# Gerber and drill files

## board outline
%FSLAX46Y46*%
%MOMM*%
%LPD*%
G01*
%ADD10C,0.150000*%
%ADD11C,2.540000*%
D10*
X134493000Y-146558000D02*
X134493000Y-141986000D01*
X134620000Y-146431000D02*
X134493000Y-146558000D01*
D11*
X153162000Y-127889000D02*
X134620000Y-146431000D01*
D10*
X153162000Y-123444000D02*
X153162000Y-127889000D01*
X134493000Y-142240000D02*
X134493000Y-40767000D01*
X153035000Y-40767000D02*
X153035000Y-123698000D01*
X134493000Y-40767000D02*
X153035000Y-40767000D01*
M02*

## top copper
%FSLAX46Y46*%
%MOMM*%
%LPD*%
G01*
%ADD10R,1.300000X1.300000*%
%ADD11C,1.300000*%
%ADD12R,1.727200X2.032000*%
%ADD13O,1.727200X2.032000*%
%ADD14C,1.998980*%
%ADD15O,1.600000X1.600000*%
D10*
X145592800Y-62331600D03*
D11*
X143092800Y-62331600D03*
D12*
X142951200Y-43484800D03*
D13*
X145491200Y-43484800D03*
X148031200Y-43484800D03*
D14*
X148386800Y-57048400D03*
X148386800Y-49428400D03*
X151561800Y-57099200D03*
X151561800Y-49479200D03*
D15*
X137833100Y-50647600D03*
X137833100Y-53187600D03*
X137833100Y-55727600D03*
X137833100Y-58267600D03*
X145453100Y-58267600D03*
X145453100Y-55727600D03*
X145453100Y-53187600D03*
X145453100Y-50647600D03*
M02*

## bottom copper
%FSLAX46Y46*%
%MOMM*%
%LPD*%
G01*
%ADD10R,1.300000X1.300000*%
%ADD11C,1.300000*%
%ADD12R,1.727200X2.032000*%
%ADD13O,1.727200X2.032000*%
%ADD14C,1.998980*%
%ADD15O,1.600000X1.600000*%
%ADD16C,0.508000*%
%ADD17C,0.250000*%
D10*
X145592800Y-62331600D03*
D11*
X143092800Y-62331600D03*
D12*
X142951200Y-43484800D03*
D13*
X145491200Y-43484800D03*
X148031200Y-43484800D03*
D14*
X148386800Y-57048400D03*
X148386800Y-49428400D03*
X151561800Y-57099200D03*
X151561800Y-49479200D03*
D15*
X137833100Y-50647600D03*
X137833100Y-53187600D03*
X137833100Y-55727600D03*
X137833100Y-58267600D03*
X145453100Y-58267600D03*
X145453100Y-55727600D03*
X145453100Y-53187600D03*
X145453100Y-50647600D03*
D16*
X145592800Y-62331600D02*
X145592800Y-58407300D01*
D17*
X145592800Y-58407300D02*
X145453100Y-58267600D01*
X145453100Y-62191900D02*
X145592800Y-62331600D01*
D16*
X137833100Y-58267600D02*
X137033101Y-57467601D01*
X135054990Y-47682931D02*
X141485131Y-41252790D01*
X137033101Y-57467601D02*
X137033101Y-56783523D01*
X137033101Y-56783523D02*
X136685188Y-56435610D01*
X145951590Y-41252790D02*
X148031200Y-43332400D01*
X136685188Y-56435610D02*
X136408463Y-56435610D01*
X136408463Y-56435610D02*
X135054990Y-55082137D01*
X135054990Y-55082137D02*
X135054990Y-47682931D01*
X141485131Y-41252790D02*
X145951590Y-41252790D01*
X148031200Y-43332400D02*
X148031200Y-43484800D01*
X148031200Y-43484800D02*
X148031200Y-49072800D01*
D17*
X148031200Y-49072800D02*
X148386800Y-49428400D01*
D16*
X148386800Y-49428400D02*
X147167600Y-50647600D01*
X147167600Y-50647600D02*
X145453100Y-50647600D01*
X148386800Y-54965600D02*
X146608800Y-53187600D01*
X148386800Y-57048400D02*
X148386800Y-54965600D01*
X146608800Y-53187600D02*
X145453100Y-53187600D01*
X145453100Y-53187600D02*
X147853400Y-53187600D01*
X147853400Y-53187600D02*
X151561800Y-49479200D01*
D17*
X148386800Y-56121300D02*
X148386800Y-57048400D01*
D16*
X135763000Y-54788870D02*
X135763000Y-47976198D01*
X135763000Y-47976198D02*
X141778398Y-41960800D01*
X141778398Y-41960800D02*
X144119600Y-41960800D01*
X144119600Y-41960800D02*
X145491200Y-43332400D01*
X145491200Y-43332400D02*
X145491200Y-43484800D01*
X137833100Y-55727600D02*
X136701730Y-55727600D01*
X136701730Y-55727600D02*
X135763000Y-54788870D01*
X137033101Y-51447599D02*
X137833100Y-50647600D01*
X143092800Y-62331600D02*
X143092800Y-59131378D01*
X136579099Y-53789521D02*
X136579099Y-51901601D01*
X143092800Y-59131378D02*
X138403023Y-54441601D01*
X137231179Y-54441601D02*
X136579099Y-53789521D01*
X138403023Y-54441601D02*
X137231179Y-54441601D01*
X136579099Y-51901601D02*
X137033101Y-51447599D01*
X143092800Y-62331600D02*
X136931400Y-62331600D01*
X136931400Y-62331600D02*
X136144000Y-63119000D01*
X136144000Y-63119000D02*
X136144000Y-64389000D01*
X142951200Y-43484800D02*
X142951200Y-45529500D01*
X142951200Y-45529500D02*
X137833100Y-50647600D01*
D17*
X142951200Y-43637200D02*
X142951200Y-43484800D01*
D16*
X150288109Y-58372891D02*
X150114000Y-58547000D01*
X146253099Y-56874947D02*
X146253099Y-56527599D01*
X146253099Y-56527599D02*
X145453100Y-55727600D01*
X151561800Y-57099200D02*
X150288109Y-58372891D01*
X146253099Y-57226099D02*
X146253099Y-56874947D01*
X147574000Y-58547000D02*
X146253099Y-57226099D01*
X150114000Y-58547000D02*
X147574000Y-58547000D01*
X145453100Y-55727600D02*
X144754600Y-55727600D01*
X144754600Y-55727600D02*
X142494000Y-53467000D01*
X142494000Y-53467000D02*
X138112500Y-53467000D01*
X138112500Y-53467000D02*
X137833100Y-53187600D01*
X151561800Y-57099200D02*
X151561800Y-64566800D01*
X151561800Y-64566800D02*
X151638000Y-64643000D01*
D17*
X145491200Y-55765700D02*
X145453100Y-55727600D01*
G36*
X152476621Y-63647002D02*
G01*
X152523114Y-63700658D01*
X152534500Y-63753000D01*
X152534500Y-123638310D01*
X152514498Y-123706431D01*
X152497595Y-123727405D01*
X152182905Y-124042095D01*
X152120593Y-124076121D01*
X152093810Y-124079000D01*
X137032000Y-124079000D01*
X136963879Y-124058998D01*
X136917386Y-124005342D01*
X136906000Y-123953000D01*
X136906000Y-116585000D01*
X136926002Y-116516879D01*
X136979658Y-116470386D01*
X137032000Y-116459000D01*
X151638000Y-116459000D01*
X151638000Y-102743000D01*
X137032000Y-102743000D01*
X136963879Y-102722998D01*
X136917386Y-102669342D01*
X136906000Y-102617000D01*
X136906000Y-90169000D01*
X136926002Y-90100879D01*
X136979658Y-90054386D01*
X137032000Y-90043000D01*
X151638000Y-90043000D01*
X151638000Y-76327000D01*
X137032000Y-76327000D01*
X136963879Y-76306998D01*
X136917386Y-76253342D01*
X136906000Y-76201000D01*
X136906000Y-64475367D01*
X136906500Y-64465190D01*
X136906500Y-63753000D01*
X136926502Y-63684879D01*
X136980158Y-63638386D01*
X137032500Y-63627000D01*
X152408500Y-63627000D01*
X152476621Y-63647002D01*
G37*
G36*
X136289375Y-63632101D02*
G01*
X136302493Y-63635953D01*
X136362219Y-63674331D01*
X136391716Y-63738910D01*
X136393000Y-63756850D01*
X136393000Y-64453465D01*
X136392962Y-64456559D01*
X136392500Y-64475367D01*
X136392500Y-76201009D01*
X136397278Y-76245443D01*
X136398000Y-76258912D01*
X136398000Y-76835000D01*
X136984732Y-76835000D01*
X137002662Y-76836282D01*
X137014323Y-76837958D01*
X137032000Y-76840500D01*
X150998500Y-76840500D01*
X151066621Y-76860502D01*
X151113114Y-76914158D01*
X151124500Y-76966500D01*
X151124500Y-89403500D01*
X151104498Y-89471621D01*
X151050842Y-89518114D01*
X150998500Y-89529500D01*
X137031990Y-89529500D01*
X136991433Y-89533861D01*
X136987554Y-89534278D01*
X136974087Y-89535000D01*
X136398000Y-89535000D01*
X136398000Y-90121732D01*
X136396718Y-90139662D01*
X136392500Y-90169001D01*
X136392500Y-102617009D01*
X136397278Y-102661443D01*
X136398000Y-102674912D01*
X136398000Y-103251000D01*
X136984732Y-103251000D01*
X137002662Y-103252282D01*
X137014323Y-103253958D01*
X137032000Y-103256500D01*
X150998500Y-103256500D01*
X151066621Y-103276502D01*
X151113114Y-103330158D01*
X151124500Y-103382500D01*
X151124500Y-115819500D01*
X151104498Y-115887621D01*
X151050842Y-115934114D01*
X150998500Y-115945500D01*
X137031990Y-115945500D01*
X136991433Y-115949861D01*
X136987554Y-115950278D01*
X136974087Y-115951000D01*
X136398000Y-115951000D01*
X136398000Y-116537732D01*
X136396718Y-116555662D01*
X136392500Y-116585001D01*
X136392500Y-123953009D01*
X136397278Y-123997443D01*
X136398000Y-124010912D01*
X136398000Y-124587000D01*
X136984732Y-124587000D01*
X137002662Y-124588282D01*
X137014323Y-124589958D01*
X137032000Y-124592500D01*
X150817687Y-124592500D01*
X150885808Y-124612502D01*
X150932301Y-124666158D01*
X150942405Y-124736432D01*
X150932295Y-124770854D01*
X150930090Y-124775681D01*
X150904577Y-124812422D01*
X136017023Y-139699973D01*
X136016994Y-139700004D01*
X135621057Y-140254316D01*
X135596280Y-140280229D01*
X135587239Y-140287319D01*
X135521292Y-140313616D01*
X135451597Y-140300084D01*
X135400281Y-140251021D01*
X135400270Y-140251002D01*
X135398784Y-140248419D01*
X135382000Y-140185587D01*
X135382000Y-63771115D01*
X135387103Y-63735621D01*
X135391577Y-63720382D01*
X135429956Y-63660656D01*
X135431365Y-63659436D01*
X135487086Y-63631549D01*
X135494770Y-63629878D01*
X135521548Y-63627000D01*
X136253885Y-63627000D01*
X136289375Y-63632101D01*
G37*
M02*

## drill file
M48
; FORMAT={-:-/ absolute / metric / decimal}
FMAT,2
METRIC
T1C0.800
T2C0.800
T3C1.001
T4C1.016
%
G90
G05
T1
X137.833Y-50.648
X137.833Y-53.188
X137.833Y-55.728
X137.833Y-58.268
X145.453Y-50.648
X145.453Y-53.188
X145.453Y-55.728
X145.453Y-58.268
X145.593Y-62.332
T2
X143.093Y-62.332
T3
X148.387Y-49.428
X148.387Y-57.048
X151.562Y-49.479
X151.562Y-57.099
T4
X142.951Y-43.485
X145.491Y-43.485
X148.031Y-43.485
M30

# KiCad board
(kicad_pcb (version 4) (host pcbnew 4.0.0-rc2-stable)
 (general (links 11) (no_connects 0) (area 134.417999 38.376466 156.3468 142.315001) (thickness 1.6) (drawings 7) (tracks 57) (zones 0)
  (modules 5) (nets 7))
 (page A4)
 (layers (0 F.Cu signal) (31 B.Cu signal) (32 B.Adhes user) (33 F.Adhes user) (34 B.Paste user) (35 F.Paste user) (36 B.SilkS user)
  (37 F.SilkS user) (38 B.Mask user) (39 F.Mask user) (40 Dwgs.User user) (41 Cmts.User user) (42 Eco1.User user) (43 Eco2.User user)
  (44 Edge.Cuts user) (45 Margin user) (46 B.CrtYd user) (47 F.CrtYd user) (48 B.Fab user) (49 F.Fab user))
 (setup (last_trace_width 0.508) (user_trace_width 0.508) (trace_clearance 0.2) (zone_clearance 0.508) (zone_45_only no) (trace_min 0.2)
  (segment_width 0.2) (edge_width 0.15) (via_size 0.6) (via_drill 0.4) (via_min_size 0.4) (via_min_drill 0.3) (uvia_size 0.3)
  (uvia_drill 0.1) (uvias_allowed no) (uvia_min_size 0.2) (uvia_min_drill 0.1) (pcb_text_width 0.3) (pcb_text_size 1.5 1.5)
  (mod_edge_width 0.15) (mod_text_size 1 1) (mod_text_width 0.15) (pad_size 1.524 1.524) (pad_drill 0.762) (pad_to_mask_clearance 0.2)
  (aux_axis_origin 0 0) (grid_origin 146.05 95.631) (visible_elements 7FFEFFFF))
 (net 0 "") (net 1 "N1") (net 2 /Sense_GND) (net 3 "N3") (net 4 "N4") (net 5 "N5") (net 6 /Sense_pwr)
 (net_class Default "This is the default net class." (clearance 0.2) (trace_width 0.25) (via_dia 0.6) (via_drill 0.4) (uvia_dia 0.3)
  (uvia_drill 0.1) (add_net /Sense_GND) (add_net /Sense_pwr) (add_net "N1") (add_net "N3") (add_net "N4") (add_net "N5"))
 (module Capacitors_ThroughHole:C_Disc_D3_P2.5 (layer F.Cu) (at 145.5928 62.3316 180)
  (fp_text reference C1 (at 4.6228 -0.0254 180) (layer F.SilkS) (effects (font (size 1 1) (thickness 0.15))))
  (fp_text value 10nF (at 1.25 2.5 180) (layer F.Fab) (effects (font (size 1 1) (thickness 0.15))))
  (pad 1 thru_hole rect (at 0 0 180) (size 1.3 1.3) (drill 0.8) (layers *.Cu *.Mask F.SilkS) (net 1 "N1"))
  (pad 2 thru_hole circle (at 2.5 0 180) (size 1.3 1.3) (drill 0.8001) (layers *.Cu *.Mask F.SilkS) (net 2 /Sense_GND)))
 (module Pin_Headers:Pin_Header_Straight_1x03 (layer F.Cu) (at 142.9512 43.4848 90)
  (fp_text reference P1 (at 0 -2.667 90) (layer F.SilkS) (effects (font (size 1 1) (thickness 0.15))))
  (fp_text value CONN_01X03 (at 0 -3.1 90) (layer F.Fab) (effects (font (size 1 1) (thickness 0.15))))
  (pad 1 thru_hole rect (at 0 0 90) (size 2.032 1.7272) (drill 1.016) (layers *.Cu *.Mask F.SilkS) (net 2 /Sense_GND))
  (pad 2 thru_hole oval (at 0 2.54 90) (size 2.032 1.7272) (drill 1.016) (layers *.Cu *.Mask F.SilkS) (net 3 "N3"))
  (pad 3 thru_hole oval (at 0 5.08 90) (size 2.032 1.7272) (drill 1.016) (layers *.Cu *.Mask F.SilkS) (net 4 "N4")))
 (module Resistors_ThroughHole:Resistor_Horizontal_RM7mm (layer F.Cu) (at 148.3868 57.0484 90)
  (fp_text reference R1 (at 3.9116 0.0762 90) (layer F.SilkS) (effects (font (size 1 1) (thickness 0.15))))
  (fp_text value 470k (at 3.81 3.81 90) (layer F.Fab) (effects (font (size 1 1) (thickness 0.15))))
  (pad 1 thru_hole circle (at 0 0 90) (size 1.99898 1.99898) (drill 1.00076) (layers *.Cu *.SilkS *.Mask) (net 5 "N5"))
  (pad 2 thru_hole circle (at 7.62 0 90) (size 1.99898 1.99898) (drill 1.00076) (layers *.Cu *.SilkS *.Mask) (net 4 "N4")))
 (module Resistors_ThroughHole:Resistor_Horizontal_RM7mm (layer F.Cu) (at 151.5618 57.0992 90)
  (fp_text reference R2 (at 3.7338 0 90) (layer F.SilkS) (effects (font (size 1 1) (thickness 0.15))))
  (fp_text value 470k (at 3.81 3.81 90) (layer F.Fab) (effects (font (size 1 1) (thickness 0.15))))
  (pad 1 thru_hole circle (at 0 0 90) (size 1.99898 1.99898) (drill 1.00076) (layers *.Cu *.SilkS *.Mask) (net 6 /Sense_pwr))
  (pad 2 thru_hole circle (at 7.62 0 90) (size 1.99898 1.99898) (drill 1.00076) (layers *.Cu *.SilkS *.Mask) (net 5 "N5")))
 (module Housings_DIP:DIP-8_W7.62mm (layer F.Cu) (at 137.8331 50.6476)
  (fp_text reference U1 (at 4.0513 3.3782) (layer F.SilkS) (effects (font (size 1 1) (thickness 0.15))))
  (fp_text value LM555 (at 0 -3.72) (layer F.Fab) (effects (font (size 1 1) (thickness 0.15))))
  (pad 1 thru_hole oval (at 0 0) (size 1.6 1.6) (drill 0.8) (layers *.Cu *.Mask F.SilkS) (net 2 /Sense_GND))
  (pad 2 thru_hole oval (at 0 2.54) (size 1.6 1.6) (drill 0.8) (layers *.Cu *.Mask F.SilkS) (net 6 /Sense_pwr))
  (pad 3 thru_hole oval (at 0 5.08) (size 1.6 1.6) (drill 0.8) (layers *.Cu *.Mask F.SilkS) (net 3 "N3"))
  (pad 4 thru_hole oval (at 0 7.62) (size 1.6 1.6) (drill 0.8) (layers *.Cu *.Mask F.SilkS) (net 4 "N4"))
  (pad 5 thru_hole oval (at 7.62 7.62) (size 1.6 1.6) (drill 0.8) (layers *.Cu *.Mask F.SilkS) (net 1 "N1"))
  (pad 6 thru_hole oval (at 7.62 5.08) (size 1.6 1.6) (drill 0.8) (layers *.Cu *.Mask F.SilkS) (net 6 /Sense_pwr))
  (pad 7 thru_hole oval (at 7.62 2.54) (size 1.6 1.6) (drill 0.8) (layers *.Cu *.Mask F.SilkS) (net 5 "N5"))
  (pad 8 thru_hole oval (at 7.62 0) (size 1.6 1.6) (drill 0.8) (layers *.Cu *.Mask F.SilkS) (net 4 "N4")))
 (gr_line (start 134.493 146.558) (end 134.493 141.986) (angle 90) (layer Edge.Cuts) (width 0.15))
 (gr_line (start 134.62 146.431) (end 134.493 146.558) (angle 90) (layer Edge.Cuts) (width 0.15))
 (gr_line (start 153.162 127.889) (end 134.62 146.431) (angle 90) (layer Edge.Cuts) (width 2.54))
 (gr_line (start 153.162 123.444) (end 153.162 127.889) (angle 90) (layer Edge.Cuts) (width 0.15))
 (gr_line (start 134.493 142.24) (end 134.493 40.767) (angle 90) (layer Edge.Cuts) (width 0.15))
 (gr_line (start 153.035 40.767) (end 153.035 123.698) (angle 90) (layer Edge.Cuts) (width 0.15))
 (gr_line (start 134.493 40.767) (end 153.035 40.767) (angle 90) (layer Edge.Cuts) (width 0.15))
 (segment (start 145.5928 62.3316) (end 145.5928 58.4073) (width 0.508) (layer B.Cu) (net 1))
 (segment (start 145.5928 58.4073) (end 145.4531 58.2676) (width 0.25) (layer B.Cu) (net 1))
 (segment (start 145.4531 62.1919) (end 145.5928 62.3316) (width 0.25) (layer B.Cu) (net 1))
 (segment (start 137.8331 58.2676) (end 137.033101 57.467601) (width 0.508) (layer B.Cu) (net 4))
 (segment (start 135.05499 47.682931) (end 141.485131 41.25279) (width 0.508) (layer B.Cu) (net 4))
 (segment (start 137.033101 57.467601) (end 137.033101 56.783523) (width 0.508) (layer B.Cu) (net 4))
 (segment (start 137.033101 56.783523) (end 136.685188 56.43561) (width 0.508) (layer B.Cu) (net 4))
 (segment (start 145.95159 41.25279) (end 148.0312 43.3324) (width 0.508) (layer B.Cu) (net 4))
 (segment (start 136.685188 56.43561) (end 136.408463 56.43561) (width 0.508) (layer B.Cu) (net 4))
 (segment (start 136.408463 56.43561) (end 135.05499 55.082137) (width 0.508) (layer B.Cu) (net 4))
 (segment (start 135.05499 55.082137) (end 135.05499 47.682931) (width 0.508) (layer B.Cu) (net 4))
 (segment (start 141.485131 41.25279) (end 145.95159 41.25279) (width 0.508) (layer B.Cu) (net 4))
 (segment (start 148.0312 43.3324) (end 148.0312 43.4848) (width 0.508) (layer B.Cu) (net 4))
 (segment (start 148.0312 43.4848) (end 148.0312 49.0728) (width 0.508) (layer B.Cu) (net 4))
 (segment (start 148.0312 49.0728) (end 148.3868 49.4284) (width 0.25) (layer B.Cu) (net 4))
 (segment (start 148.3868 49.4284) (end 147.1676 50.6476) (width 0.508) (layer B.Cu) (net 4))
 (segment (start 147.1676 50.6476) (end 145.4531 50.6476) (width 0.508) (layer B.Cu) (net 4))
 (segment (start 148.3868 54.9656) (end 146.6088 53.1876) (width 0.508) (layer B.Cu) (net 5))
 (segment (start 148.3868 57.0484) (end 148.3868 54.9656) (width 0.508) (layer B.Cu) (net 5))
 (segment (start 146.6088 53.1876) (end 145.4531 53.1876) (width 0.508) (layer B.Cu) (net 5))
 (segment (start 145.4531 53.1876) (end 147.8534 53.1876) (width 0.508) (layer B.Cu) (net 5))
 (segment (start 147.8534 53.1876) (end 151.5618 49.4792) (width 0.508) (layer B.Cu) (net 5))
 (segment (start 148.3868 56.1213) (end 148.3868 57.0484) (width 0.25) (layer B.Cu) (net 5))
 (segment (start 135.763 54.78887) (end 135.763 47.976198) (width 0.508) (layer B.Cu) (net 3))
 (segment (start 135.763 47.976198) (end 141.778398 41.9608) (width 0.508) (layer B.Cu) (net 3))
 (segment (start 141.778398 41.9608) (end 144.1196 41.9608) (width 0.508) (layer B.Cu) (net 3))
 (segment (start 144.1196 41.9608) (end 145.4912 43.3324) (width 0.508) (layer B.Cu) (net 3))
 (segment (start 145.4912 43.3324) (end 145.4912 43.4848) (width 0.508) (layer B.Cu) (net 3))
 (segment (start 137.8331 55.7276) (end 136.70173 55.7276) (width 0.508) (layer B.Cu) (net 3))
 (segment (start 136.70173 55.7276) (end 135.763 54.78887) (width 0.508) (layer B.Cu) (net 3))
 (segment (start 137.033101 51.447599) (end 137.8331 50.6476) (width 0.508) (layer B.Cu) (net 2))
 (segment (start 143.0928 62.3316) (end 143.0928 59.131378) (width 0.508) (layer B.Cu) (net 2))
 (segment (start 136.579099 53.789521) (end 136.579099 51.901601) (width 0.508) (layer B.Cu) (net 2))
 (segment (start 143.0928 59.131378) (end 138.403023 54.441601) (width 0.508) (layer B.Cu) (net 2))
 (segment (start 137.231179 54.441601) (end 136.579099 53.789521) (width 0.508) (layer B.Cu) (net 2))
 (segment (start 138.403023 54.441601) (end 137.231179 54.441601) (width 0.508) (layer B.Cu) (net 2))
 (segment (start 136.579099 51.901601) (end 137.033101 51.447599) (width 0.508) (layer B.Cu) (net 2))
 (segment (start 143.0928 62.3316) (end 136.9314 62.3316) (width 0.508) (layer B.Cu) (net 2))
 (segment (start 136.9314 62.3316) (end 136.144 63.119) (width 0.508) (layer B.Cu) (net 2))
 (segment (start 136.144 63.119) (end 136.144 64.389) (width 0.508) (layer B.Cu) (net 2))
 (segment (start 142.9512 43.4848) (end 142.9512 45.5295) (width 0.508) (layer B.Cu) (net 2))
 (segment (start 142.9512 45.5295) (end 137.8331 50.6476) (width 0.508) (layer B.Cu) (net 2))
 (segment (start 142.9512 43.6372) (end 142.9512 43.4848) (width 0.25) (layer B.Cu) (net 2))
 (segment (start 150.288109 58.372891) (end 150.114 58.547) (width 0.508) (layer B.Cu) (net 6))
 (segment (start 146.253099 56.874947) (end 146.253099 56.527599) (width 0.508) (layer B.Cu) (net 6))
 (segment (start 146.253099 56.527599) (end 145.4531 55.7276) (width 0.508) (layer B.Cu) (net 6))
 (segment (start 151.5618 57.0992) (end 150.288109 58.372891) (width 0.508) (layer B.Cu) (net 6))
 (segment (start 146.253099 57.226099) (end 146.253099 56.874947) (width 0.508) (layer B.Cu) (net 6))
 (segment (start 147.574 58.547) (end 146.253099 57.226099) (width 0.508) (layer B.Cu) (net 6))
 (segment (start 150.114 58.547) (end 147.574 58.547) (width 0.508) (layer B.Cu) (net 6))
 (segment (start 145.4531 55.7276) (end 144.7546 55.7276) (width 0.508) (layer B.Cu) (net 6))
 (segment (start 144.7546 55.7276) (end 142.494 53.467) (width 0.508) (layer B.Cu) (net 6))
 (segment (start 142.494 53.467) (end 138.1125 53.467) (width 0.508) (layer B.Cu) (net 6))
 (segment (start 138.1125 53.467) (end 137.8331 53.1876) (width 0.508) (layer B.Cu) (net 6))
 (segment (start 151.5618 57.0992) (end 151.5618 64.5668) (width 0.508) (layer B.Cu) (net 6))
 (segment (start 151.5618 64.5668) (end 151.638 64.643) (width 0.508) (layer B.Cu) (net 6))
 (segment (start 145.4912 55.7657) (end 145.4531 55.7276) (width 0.25) (layer B.Cu) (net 6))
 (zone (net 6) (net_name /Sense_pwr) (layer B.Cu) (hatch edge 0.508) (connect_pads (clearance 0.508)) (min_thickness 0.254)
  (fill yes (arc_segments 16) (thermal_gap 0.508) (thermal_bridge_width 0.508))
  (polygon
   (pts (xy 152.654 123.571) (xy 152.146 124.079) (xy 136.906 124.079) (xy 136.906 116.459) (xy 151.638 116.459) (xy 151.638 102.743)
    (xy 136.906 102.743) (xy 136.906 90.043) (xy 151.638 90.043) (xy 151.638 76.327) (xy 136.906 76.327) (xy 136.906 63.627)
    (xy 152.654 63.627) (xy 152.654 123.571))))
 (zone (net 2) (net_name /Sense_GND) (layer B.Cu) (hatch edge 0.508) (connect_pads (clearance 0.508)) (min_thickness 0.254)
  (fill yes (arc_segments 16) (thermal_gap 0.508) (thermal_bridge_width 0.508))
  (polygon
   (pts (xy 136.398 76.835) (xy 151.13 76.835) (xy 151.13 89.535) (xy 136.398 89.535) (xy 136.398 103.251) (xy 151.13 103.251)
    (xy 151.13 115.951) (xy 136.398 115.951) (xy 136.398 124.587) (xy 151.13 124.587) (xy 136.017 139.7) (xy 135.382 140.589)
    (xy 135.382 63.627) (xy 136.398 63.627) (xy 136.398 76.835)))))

